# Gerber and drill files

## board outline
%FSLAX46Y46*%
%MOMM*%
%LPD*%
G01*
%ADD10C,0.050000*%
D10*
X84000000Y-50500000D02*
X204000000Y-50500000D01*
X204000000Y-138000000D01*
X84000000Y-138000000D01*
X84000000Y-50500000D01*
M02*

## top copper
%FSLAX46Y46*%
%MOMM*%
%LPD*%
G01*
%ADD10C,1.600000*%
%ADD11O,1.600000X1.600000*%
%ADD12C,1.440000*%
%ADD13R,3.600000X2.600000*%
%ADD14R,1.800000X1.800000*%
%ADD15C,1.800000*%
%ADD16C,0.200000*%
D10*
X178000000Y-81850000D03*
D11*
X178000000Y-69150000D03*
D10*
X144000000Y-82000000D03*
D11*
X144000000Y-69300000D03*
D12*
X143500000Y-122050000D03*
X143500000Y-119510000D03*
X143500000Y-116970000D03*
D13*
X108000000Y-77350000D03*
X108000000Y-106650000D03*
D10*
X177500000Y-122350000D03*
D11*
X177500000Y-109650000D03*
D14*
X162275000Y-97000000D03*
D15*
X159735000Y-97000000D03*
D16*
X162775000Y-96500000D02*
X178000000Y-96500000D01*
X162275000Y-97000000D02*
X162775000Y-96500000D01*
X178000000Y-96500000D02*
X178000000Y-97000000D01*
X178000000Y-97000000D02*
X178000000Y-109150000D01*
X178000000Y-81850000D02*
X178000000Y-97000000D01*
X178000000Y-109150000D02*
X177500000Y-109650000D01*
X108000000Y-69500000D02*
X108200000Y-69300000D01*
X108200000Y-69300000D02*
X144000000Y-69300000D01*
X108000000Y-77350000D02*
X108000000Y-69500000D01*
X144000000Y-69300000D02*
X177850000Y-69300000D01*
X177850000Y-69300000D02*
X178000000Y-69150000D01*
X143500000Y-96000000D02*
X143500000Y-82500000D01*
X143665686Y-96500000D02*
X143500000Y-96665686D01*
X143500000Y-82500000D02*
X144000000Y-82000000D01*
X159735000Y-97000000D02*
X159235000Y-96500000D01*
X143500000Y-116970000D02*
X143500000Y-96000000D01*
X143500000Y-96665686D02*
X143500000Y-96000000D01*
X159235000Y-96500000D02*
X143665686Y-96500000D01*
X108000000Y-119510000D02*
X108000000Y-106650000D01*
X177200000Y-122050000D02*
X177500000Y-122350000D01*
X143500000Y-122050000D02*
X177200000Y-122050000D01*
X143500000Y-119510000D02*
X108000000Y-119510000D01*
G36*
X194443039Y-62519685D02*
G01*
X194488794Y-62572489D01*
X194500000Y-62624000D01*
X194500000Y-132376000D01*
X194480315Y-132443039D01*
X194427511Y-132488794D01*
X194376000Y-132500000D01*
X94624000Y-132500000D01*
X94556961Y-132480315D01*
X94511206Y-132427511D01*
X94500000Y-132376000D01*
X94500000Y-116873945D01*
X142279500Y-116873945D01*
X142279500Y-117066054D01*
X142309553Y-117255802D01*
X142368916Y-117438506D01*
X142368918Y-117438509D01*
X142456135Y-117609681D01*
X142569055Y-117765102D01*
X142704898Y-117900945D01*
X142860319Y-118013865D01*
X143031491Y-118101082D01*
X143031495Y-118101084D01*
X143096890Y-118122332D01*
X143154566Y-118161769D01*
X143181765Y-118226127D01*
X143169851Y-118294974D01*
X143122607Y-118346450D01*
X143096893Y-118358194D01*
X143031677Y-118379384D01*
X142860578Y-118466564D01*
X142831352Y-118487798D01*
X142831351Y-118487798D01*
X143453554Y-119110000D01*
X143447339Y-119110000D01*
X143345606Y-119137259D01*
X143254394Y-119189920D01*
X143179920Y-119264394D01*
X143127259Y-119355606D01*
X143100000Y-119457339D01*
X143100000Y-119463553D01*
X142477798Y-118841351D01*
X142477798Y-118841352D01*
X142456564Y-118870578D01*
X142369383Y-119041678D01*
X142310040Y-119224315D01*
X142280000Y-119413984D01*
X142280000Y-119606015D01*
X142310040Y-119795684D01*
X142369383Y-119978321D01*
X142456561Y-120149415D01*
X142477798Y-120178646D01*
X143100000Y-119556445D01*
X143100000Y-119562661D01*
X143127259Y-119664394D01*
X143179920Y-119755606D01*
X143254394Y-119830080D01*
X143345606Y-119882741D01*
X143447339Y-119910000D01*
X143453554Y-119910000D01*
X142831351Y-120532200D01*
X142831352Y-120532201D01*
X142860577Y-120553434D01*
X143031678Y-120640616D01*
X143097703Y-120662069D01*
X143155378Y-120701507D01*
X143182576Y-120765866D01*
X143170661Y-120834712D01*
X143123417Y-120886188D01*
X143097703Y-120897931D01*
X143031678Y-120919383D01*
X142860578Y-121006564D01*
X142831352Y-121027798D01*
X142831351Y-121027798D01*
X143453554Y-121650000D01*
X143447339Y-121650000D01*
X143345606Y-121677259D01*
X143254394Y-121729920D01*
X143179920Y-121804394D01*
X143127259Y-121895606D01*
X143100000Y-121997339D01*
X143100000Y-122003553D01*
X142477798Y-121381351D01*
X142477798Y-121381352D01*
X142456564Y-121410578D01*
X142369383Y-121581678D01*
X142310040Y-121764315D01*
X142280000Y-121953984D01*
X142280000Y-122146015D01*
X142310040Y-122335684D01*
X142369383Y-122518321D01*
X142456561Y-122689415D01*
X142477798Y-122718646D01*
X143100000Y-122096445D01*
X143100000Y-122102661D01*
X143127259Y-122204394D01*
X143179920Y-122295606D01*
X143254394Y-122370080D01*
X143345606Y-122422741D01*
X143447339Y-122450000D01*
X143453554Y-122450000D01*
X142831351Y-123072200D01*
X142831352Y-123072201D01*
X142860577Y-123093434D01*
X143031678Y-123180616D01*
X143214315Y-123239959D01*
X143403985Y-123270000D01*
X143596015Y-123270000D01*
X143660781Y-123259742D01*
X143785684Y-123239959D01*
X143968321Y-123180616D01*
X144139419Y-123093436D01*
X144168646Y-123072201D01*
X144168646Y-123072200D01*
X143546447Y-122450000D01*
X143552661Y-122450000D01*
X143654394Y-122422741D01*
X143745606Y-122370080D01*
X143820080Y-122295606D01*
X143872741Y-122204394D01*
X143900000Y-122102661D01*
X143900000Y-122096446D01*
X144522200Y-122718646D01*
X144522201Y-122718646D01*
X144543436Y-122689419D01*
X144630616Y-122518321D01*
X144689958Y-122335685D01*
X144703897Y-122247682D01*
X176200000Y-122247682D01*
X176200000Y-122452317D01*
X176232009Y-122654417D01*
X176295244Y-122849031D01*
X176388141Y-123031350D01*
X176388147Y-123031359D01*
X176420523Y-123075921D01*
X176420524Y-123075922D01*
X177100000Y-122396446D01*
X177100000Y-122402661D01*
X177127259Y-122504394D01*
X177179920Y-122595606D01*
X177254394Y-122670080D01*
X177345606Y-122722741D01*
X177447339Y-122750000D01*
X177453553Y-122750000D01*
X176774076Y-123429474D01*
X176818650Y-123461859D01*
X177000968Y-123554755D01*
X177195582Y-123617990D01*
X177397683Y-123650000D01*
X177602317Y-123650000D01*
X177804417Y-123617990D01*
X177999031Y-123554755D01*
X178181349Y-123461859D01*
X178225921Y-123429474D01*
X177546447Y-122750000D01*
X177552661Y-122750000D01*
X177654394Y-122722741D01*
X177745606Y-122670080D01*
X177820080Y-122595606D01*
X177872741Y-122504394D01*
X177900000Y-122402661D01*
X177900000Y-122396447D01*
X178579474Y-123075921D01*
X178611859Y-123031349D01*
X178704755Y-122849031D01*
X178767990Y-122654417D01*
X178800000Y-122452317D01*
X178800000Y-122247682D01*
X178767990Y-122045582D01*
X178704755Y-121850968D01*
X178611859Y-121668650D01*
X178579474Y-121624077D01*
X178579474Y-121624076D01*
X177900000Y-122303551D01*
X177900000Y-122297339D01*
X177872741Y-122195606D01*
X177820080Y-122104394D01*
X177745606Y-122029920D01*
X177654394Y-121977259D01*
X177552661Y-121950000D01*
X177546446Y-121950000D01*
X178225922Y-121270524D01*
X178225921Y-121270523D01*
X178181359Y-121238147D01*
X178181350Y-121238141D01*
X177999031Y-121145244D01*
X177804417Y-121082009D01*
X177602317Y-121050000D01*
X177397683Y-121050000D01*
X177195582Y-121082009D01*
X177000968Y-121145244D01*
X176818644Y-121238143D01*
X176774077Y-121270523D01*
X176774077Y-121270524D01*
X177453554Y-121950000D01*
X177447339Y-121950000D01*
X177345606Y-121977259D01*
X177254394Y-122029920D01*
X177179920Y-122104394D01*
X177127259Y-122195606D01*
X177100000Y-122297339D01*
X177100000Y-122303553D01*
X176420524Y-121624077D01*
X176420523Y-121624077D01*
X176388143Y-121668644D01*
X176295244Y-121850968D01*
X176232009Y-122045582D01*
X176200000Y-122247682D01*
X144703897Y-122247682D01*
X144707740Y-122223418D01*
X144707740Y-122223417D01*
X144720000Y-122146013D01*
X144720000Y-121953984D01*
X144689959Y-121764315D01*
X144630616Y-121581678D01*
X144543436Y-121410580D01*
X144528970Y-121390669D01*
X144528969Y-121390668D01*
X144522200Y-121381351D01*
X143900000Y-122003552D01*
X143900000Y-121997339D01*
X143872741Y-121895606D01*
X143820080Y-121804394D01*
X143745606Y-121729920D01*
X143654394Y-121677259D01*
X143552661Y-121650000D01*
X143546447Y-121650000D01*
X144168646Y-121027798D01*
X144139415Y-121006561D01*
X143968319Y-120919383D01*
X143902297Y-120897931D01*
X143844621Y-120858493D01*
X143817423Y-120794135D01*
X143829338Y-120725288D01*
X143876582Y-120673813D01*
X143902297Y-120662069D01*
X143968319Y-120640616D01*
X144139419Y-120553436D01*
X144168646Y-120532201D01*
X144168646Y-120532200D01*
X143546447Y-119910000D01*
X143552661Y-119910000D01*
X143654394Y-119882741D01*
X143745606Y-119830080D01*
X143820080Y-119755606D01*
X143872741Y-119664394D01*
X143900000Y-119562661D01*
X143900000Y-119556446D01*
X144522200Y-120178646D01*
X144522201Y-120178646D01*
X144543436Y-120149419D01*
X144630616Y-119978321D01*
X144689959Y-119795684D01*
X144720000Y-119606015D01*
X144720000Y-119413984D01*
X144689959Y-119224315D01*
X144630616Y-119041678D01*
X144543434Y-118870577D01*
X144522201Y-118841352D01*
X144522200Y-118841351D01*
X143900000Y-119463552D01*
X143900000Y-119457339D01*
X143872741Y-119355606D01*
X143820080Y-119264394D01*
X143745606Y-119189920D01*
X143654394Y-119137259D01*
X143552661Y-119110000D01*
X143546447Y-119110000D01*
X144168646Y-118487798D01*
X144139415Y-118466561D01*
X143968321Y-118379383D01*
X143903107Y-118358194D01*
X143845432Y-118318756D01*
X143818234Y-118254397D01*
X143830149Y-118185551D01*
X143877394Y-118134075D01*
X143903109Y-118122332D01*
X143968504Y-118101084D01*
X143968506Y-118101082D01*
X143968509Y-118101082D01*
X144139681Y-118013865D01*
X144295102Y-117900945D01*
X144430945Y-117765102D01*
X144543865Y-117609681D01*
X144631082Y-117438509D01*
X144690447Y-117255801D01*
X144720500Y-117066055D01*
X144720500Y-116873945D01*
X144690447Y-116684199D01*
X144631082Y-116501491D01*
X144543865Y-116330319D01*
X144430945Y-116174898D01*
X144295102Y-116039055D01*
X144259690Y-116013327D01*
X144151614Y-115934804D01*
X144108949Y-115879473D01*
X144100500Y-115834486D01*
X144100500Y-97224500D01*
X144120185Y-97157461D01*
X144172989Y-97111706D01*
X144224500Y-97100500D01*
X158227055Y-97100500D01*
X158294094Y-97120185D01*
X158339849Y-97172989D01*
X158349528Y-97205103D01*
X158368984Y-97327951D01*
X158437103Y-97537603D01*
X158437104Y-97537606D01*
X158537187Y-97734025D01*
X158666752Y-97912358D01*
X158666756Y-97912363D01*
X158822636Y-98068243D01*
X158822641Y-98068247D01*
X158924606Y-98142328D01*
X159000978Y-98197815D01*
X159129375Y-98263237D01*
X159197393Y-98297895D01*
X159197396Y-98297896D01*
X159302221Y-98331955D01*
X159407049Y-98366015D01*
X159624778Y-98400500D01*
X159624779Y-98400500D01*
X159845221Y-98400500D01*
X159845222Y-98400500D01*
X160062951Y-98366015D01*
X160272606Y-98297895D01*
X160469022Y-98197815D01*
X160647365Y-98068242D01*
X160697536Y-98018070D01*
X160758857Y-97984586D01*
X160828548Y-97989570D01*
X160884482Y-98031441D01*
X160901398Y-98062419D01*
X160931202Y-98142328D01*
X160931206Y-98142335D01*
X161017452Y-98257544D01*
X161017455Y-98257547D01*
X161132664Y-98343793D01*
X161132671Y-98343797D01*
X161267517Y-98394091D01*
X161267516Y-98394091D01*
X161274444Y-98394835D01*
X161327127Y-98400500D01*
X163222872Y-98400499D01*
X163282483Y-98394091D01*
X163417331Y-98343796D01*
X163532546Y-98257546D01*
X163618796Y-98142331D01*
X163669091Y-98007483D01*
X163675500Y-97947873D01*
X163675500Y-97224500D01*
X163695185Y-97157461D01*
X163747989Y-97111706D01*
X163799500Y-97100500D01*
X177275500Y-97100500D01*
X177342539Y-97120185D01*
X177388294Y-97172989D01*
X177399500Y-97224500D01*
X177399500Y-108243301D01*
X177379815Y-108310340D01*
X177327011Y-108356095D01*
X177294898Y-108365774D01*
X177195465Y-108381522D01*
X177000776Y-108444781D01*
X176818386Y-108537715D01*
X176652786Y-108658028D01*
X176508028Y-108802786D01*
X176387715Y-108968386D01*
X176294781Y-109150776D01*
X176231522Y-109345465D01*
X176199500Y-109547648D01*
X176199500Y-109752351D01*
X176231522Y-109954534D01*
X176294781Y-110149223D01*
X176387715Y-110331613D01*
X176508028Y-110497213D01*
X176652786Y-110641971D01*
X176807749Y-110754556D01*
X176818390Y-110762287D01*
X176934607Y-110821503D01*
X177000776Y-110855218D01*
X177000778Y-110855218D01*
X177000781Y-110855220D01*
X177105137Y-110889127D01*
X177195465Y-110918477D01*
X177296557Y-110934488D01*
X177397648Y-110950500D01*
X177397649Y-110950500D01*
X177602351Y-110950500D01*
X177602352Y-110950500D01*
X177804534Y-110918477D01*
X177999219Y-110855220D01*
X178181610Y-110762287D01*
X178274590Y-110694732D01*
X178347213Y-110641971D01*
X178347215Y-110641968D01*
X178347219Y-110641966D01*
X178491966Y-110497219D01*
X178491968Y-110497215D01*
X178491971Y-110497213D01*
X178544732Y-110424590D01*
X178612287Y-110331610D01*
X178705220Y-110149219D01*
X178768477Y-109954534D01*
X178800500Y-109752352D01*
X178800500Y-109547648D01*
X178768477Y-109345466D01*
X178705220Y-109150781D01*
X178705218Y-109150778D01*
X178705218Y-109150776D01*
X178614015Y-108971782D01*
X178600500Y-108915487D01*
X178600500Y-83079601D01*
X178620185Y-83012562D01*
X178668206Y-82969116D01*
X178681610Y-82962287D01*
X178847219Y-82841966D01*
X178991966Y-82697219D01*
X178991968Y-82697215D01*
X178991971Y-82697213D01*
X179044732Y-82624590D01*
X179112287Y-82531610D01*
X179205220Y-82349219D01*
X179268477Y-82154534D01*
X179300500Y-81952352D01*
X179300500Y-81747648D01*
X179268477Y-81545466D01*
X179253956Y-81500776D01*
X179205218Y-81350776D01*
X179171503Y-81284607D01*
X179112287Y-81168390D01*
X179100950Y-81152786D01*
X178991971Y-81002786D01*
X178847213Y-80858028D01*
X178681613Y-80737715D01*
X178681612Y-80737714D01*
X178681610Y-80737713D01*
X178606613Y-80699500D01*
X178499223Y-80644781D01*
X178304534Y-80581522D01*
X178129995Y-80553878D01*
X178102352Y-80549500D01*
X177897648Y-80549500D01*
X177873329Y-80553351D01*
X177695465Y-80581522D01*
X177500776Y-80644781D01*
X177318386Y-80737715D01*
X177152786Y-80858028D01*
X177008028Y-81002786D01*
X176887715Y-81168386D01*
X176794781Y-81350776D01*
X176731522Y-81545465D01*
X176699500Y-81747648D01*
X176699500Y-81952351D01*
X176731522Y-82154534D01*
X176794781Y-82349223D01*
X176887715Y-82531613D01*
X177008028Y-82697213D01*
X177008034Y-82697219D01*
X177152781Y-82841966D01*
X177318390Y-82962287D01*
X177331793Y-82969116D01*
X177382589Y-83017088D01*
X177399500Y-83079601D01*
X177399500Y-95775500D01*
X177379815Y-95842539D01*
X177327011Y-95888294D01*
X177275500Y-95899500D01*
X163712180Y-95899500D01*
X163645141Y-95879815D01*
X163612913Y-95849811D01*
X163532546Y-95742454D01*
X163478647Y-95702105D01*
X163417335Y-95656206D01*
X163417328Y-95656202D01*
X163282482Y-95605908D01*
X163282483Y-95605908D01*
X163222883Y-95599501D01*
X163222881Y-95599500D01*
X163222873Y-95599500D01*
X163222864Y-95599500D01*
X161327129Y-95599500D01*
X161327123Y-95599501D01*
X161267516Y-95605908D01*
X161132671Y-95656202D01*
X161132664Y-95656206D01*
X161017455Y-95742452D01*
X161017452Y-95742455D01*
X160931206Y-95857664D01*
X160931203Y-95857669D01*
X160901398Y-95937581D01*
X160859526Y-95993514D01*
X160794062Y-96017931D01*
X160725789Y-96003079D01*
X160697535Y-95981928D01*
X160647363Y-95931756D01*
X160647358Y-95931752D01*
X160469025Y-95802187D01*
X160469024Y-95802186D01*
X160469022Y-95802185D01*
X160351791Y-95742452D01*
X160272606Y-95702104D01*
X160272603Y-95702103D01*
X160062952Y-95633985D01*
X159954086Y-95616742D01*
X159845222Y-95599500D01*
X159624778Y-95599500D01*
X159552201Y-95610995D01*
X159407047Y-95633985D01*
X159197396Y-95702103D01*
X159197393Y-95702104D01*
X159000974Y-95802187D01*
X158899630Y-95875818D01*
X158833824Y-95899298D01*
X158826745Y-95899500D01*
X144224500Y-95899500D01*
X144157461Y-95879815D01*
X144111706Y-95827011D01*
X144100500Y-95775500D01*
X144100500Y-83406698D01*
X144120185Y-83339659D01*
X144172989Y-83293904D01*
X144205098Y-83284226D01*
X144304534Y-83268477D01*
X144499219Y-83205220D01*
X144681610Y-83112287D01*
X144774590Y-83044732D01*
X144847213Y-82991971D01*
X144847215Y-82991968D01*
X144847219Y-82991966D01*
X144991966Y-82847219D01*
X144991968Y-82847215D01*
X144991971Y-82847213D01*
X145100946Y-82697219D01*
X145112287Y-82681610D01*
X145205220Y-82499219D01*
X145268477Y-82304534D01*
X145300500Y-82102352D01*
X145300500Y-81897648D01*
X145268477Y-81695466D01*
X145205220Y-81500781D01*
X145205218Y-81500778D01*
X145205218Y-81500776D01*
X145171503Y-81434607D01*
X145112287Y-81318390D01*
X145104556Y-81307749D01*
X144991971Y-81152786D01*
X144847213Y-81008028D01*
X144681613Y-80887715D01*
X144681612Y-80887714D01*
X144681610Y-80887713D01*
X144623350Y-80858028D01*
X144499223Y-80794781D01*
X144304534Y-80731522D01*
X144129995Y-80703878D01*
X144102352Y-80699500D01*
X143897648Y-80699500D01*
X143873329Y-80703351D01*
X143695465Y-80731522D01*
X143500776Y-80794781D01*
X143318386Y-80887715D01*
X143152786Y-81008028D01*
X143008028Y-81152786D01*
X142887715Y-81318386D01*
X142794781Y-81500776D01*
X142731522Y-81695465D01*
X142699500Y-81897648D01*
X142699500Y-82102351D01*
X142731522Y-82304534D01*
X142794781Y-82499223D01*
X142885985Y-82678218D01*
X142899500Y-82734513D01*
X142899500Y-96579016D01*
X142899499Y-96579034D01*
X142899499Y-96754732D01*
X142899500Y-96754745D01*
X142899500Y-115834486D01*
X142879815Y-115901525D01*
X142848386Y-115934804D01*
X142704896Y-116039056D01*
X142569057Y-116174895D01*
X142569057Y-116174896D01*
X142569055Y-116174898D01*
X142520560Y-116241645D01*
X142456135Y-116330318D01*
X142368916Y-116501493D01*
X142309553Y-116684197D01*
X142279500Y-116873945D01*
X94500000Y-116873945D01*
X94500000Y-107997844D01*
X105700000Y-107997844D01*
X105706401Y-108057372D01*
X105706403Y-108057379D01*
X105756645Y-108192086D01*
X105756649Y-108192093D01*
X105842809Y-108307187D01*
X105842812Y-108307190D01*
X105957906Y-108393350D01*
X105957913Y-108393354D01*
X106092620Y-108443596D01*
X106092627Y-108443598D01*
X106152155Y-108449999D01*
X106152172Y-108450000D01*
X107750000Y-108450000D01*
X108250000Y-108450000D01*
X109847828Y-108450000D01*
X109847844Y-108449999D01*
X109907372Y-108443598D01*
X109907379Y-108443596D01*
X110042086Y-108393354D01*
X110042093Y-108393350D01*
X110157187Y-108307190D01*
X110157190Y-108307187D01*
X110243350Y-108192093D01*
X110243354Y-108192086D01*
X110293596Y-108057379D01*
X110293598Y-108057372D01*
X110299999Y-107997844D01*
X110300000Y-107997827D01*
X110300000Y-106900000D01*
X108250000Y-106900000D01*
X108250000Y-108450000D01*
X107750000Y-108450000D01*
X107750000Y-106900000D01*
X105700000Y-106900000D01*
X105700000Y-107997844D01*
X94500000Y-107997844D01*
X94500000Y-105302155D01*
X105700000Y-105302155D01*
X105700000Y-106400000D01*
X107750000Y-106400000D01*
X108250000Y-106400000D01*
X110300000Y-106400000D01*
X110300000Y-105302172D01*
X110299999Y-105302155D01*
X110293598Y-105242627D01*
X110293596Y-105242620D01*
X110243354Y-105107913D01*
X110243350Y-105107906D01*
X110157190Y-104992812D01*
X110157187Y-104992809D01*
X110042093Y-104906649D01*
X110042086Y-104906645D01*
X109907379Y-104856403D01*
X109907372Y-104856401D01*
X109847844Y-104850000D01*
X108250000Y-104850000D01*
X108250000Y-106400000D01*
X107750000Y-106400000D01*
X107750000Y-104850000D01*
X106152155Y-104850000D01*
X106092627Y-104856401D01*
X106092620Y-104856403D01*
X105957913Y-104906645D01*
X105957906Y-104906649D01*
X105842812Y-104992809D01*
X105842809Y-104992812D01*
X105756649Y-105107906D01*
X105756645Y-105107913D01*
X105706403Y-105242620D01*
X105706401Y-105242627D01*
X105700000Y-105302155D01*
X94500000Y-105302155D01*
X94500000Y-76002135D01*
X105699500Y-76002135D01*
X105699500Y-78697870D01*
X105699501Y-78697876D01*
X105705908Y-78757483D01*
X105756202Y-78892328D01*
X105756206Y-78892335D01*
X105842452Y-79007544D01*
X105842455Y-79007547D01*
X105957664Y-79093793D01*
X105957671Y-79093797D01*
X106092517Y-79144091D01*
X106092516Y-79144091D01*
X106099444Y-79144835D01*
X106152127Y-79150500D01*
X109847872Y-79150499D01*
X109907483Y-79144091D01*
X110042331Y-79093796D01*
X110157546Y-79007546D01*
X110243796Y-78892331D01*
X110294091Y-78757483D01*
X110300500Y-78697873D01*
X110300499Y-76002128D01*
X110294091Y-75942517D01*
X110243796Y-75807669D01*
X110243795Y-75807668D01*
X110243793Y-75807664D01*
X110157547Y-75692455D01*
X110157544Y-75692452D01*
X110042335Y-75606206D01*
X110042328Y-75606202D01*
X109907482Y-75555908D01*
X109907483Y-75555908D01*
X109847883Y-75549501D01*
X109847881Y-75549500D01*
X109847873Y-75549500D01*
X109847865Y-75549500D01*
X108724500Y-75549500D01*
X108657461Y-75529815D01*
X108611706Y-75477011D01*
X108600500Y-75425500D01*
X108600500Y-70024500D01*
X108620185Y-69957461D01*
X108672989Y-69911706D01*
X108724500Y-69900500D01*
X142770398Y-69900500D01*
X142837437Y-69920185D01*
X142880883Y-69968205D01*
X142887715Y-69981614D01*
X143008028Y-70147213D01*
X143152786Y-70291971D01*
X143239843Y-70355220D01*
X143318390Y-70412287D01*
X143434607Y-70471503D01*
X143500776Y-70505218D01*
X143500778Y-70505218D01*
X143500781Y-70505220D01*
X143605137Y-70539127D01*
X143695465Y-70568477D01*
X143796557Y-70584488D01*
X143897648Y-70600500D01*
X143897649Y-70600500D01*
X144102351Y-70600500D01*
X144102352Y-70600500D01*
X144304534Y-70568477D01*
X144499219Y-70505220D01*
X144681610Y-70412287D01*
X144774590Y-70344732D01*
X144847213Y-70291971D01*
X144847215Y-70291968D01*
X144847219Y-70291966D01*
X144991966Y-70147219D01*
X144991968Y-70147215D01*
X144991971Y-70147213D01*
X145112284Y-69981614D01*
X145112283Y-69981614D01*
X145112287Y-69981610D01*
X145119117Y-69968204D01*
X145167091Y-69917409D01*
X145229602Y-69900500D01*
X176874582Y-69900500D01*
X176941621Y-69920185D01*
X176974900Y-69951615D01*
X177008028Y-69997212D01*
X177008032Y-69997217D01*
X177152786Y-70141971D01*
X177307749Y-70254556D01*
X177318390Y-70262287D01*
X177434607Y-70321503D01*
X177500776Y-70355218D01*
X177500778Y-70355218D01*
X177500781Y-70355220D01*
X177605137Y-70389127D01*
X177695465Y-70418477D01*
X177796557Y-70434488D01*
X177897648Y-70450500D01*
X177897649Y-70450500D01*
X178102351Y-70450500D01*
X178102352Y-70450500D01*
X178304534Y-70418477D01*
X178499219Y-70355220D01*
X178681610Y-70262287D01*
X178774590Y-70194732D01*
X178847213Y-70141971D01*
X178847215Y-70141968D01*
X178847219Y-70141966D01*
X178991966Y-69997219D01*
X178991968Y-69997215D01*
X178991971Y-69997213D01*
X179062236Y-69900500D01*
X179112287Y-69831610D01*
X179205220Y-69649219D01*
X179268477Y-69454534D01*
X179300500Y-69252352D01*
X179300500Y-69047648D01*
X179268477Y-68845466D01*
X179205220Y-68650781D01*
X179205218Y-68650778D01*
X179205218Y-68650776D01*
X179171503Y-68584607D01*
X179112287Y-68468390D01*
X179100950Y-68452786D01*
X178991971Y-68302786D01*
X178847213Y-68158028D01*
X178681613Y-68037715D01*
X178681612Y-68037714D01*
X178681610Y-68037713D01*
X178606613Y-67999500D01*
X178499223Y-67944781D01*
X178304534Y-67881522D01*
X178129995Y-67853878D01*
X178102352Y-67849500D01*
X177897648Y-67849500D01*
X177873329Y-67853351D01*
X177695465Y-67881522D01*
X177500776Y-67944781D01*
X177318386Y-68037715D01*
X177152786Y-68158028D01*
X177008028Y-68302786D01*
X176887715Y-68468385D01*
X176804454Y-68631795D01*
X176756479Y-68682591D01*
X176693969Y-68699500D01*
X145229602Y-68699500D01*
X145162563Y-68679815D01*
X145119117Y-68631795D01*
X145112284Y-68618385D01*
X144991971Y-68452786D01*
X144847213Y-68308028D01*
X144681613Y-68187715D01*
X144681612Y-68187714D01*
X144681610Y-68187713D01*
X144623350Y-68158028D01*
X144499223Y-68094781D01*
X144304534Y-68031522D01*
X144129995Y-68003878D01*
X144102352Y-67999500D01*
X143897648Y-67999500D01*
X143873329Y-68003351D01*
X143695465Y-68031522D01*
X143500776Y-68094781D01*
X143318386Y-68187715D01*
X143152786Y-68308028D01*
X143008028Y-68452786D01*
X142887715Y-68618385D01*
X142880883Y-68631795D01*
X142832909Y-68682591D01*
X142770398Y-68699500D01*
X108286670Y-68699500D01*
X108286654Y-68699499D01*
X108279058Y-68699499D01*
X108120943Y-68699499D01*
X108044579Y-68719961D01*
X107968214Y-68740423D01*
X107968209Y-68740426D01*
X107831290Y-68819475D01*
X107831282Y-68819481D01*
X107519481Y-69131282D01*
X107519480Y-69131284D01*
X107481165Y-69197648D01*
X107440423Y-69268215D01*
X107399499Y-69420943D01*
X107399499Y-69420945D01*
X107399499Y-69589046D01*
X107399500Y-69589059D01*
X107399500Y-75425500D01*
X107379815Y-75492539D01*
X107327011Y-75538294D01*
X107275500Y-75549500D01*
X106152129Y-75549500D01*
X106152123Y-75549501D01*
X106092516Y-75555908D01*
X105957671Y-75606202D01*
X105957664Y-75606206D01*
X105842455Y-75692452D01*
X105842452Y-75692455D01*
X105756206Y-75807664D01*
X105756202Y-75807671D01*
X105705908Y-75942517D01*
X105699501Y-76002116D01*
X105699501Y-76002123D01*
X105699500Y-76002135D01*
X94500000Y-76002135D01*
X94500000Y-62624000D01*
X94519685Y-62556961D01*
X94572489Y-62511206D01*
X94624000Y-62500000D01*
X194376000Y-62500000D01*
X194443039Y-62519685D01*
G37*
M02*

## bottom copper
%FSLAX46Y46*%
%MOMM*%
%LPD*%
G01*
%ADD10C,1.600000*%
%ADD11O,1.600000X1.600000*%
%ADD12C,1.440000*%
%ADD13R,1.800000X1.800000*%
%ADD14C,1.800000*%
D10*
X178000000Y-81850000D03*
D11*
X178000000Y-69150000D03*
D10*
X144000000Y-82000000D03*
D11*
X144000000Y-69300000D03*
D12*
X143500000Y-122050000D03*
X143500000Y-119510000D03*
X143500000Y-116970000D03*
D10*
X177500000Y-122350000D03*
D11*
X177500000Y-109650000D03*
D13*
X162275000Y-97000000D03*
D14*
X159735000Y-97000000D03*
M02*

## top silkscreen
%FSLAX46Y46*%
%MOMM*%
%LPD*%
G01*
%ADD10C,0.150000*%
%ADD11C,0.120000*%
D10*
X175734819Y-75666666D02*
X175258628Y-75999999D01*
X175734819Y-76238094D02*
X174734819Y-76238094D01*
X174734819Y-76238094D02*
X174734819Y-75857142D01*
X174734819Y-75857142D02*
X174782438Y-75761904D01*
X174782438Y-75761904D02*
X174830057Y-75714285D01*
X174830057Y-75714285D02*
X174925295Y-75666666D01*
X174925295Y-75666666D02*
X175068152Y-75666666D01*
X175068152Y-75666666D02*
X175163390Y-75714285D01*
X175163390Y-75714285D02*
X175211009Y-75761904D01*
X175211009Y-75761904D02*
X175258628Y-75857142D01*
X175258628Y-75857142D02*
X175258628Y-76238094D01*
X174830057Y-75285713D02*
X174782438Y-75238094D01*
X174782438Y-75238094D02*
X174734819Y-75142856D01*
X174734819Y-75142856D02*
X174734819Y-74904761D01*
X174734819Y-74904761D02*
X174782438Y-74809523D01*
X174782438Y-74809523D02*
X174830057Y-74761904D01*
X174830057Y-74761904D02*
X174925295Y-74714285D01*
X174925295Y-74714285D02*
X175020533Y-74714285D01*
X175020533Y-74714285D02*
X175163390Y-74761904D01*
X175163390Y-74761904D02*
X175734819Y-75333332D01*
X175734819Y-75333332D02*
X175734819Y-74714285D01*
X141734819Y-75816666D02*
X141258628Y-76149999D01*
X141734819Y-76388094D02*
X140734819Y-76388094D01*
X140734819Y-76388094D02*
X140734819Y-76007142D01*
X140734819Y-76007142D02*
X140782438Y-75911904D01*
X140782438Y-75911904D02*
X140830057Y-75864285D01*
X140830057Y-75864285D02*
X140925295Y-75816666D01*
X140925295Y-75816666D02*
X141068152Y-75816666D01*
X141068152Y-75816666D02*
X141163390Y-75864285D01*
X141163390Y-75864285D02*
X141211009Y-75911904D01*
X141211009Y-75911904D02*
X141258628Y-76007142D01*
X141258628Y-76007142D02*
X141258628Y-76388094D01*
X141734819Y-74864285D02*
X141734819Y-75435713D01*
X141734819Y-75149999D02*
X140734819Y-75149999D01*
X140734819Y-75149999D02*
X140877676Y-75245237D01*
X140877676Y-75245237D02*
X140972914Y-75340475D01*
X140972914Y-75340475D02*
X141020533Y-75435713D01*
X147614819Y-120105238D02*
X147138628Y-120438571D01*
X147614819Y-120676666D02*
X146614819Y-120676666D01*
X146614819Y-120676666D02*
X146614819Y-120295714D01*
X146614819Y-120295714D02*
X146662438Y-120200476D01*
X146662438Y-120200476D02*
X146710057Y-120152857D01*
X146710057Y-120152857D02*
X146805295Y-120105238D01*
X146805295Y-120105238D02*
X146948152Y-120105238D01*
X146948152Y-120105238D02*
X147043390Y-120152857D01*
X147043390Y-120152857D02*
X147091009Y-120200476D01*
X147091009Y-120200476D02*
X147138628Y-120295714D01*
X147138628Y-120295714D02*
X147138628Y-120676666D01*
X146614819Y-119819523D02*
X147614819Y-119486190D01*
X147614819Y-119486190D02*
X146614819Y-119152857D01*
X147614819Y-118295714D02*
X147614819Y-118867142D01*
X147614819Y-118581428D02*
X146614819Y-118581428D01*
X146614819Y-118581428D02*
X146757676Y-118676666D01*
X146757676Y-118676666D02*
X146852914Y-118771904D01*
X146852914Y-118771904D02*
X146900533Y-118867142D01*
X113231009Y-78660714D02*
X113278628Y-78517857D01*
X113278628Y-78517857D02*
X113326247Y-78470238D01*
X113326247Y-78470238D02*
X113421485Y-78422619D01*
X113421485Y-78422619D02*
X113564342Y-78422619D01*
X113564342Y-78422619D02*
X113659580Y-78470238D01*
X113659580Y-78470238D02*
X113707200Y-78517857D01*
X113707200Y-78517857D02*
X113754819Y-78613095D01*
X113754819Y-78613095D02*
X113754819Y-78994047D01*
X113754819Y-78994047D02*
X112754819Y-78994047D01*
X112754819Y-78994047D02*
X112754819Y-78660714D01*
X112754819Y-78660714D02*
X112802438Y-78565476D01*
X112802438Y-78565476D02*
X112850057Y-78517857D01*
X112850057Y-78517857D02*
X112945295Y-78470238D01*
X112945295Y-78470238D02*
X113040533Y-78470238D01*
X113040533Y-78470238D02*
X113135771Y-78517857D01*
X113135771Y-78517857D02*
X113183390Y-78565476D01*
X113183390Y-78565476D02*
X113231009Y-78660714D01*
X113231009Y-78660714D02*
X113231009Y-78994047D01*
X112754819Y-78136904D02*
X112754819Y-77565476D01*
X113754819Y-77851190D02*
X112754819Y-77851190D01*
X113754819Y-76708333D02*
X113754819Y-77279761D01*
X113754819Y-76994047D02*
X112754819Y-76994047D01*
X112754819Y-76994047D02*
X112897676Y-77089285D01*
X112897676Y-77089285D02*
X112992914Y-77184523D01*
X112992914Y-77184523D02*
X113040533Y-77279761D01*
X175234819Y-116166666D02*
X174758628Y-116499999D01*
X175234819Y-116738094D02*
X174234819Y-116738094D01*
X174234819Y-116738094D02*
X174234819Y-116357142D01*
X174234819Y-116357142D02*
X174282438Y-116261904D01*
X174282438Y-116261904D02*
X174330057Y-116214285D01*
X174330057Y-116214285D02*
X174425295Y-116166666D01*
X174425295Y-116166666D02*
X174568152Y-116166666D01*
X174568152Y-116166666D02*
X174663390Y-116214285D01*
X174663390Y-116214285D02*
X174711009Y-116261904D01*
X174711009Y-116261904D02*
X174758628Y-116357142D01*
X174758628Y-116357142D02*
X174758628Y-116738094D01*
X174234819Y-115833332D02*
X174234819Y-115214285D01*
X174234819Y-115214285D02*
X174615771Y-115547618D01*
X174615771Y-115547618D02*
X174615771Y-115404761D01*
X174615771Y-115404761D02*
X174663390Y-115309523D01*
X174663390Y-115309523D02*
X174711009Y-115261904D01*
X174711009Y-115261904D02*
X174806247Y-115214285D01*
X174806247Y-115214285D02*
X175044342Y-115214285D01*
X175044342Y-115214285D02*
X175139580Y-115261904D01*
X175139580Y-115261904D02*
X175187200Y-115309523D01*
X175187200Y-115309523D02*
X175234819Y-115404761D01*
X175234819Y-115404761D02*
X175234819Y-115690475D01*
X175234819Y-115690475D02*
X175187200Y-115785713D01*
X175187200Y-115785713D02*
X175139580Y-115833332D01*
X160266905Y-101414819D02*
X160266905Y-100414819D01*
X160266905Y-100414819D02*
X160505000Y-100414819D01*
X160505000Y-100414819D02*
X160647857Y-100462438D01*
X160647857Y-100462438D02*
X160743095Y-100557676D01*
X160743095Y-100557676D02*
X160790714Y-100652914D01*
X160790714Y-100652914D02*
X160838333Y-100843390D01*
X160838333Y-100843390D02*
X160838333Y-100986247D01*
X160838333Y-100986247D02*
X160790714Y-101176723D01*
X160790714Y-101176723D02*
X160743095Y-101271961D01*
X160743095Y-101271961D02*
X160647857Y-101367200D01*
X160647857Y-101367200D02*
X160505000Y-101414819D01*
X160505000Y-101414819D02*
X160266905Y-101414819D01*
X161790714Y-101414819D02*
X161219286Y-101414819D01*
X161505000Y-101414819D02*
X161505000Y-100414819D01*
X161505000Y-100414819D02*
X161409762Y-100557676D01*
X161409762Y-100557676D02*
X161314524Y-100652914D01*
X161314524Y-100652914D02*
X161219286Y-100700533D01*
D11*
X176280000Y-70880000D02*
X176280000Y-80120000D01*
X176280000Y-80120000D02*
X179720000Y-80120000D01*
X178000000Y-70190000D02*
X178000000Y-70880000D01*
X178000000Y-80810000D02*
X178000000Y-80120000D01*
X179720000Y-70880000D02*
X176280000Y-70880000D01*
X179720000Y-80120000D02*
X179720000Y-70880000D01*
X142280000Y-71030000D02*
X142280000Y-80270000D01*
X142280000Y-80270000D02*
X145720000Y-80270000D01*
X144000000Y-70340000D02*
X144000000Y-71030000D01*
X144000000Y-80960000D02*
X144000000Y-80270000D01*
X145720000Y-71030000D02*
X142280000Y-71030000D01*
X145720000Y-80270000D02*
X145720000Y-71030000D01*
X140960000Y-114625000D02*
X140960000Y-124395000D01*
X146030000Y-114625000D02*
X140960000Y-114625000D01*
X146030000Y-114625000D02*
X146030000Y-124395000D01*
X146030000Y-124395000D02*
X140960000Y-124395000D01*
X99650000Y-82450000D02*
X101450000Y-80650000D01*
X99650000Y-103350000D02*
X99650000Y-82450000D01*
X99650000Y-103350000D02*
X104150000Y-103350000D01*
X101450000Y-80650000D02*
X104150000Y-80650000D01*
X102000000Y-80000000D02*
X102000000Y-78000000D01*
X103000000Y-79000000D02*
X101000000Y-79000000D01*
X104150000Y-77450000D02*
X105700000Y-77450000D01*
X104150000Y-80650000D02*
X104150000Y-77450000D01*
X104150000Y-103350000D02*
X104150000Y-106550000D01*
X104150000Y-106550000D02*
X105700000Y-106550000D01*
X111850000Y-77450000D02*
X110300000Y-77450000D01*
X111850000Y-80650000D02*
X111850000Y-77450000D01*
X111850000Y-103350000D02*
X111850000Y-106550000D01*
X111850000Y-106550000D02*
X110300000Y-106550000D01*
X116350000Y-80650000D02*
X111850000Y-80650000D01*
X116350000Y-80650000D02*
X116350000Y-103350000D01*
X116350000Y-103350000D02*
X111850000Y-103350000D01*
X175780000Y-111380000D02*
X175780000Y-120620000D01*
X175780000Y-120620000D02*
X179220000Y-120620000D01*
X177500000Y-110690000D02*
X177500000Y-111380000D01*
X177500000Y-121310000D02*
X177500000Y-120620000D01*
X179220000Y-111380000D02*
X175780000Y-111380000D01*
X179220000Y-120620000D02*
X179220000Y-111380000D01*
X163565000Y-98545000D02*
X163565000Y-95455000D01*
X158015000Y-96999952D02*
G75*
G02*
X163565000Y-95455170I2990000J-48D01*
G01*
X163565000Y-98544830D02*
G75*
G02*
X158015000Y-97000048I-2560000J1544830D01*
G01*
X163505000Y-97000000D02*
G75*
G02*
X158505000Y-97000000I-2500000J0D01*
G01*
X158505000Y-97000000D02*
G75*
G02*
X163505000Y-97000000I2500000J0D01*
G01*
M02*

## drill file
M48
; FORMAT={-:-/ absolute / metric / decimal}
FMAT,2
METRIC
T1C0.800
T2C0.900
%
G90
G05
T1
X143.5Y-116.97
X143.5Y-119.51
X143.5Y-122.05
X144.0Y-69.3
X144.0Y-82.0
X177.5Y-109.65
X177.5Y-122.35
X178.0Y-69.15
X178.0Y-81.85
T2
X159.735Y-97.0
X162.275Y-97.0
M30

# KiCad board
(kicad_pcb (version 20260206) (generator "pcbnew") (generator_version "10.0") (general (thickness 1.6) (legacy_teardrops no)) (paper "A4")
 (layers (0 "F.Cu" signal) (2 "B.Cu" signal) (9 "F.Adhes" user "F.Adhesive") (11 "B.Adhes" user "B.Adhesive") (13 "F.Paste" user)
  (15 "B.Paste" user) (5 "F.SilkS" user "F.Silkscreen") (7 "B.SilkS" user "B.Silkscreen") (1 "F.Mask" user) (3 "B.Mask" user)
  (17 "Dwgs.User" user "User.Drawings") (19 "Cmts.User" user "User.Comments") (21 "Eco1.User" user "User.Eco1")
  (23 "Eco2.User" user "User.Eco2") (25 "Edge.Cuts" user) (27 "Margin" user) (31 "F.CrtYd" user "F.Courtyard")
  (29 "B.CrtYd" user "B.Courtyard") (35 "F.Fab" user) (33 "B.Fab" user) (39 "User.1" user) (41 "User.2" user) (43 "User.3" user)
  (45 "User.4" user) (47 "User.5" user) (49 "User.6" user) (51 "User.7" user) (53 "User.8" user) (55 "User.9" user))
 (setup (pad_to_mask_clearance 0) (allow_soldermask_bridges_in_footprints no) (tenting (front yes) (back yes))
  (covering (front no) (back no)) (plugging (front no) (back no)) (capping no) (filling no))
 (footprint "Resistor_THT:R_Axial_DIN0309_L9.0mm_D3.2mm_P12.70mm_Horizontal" (layer "F.Cu") (at 178 81.85 90)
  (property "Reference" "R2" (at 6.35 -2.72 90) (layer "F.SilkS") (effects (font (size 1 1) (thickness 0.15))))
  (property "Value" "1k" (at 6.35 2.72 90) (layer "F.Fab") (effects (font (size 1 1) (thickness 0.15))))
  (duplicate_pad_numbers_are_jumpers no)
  (fp_line (start 10.97 -1.72) (end 1.73 -1.72) (stroke (width 0.12) (type solid)) (layer "F.SilkS"))
  (fp_line (start 1.73 -1.72) (end 1.73 1.72) (stroke (width 0.12) (type solid)) (layer "F.SilkS"))
  (fp_line (start 11.66 0) (end 10.97 0) (stroke (width 0.12) (type solid)) (layer "F.SilkS"))
  (fp_line (start 1.04 0) (end 1.73 0) (stroke (width 0.12) (type solid)) (layer "F.SilkS"))
  (fp_line (start 10.97 1.72) (end 10.97 -1.72) (stroke (width 0.12) (type solid)) (layer "F.SilkS"))
  (fp_line (start 1.73 1.72) (end 10.97 1.72) (stroke (width 0.12) (type solid)) (layer "F.SilkS"))
  (pad "1" thru_hole circle (at 0 0 90) (size 1.6 1.6) (drill 0.8) (layers "*.Cu" "*.Mask") (remove_unused_layers no) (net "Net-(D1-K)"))
  (pad "2" thru_hole oval (at 12.7 0 90) (size 1.6 1.6) (drill 0.8) (layers "*.Cu" "*.Mask") (remove_unused_layers no) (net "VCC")))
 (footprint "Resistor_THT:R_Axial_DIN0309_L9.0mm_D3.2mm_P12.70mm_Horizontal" (layer "F.Cu") (at 144 82 90)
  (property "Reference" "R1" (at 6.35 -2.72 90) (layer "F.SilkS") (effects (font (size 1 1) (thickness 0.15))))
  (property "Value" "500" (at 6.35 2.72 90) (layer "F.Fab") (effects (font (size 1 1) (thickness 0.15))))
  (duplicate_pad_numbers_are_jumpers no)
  (fp_line (start 10.97 -1.72) (end 1.73 -1.72) (stroke (width 0.12) (type solid)) (layer "F.SilkS"))
  (fp_line (start 1.73 -1.72) (end 1.73 1.72) (stroke (width 0.12) (type solid)) (layer "F.SilkS"))
  (fp_line (start 11.66 0) (end 10.97 0) (stroke (width 0.12) (type solid)) (layer "F.SilkS"))
  (fp_line (start 1.04 0) (end 1.73 0) (stroke (width 0.12) (type solid)) (layer "F.SilkS"))
  (fp_line (start 10.97 1.72) (end 10.97 -1.72) (stroke (width 0.12) (type solid)) (layer "F.SilkS"))
  (fp_line (start 1.73 1.72) (end 10.97 1.72) (stroke (width 0.12) (type solid)) (layer "F.SilkS"))
  (pad "1" thru_hole circle (at 0 0 90) (size 1.6 1.6) (drill 0.8) (layers "*.Cu" "*.Mask") (remove_unused_layers no) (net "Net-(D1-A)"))
  (pad "2" thru_hole oval (at 12.7 0 90) (size 1.6 1.6) (drill 0.8) (layers "*.Cu" "*.Mask") (remove_unused_layers no) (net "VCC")))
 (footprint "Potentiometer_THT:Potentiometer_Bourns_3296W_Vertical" (layer "F.Cu") (at 143.5 122.05 -90)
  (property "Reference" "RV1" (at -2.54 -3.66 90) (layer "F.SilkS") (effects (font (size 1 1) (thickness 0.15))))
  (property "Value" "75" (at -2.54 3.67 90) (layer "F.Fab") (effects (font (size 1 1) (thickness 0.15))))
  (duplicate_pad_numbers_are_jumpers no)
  (fp_line (start -7.425 2.54) (end 2.345 2.54) (stroke (width 0.12) (type solid)) (layer "F.SilkS"))
  (fp_line (start -7.425 -2.53) (end -7.425 2.54) (stroke (width 0.12) (type solid)) (layer "F.SilkS"))
  (fp_line (start -7.425 -2.53) (end 2.345 -2.53) (stroke (width 0.12) (type solid)) (layer "F.SilkS"))
  (fp_line (start 2.345 -2.53) (end 2.345 2.54) (stroke (width 0.12) (type solid)) (layer "F.SilkS"))
  (pad "1" thru_hole circle (at 0 0 270) (size 1.44 1.44) (drill 0.8) (layers "*.Cu" "*.Mask") (remove_unused_layers no) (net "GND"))
  (pad "2" thru_hole circle (at -2.54 0 270) (size 1.44 1.44) (drill 0.8) (layers "*.Cu" "*.Mask") (remove_unused_layers no) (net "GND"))
  (pad "3" thru_hole circle (at -5.08 0 270) (size 1.44 1.44) (drill 0.8) (layers "*.Cu" "*.Mask") (remove_unused_layers no)
   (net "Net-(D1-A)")))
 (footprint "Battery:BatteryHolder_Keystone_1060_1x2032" (layer "F.Cu") (at 108 92 -90)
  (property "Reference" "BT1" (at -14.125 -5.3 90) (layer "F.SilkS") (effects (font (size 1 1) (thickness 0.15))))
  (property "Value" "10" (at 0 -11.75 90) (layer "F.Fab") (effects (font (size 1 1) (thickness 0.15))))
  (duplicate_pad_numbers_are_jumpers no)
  (fp_line (start -9.55 8.35) (end -11.35 6.55) (stroke (width 0.12) (type solid)) (layer "F.SilkS"))
  (fp_line (start 11.35 8.35) (end -9.55 8.35) (stroke (width 0.12) (type solid)) (layer "F.SilkS"))
  (fp_line (start 11.35 8.35) (end 11.35 3.85) (stroke (width 0.12) (type solid)) (layer "F.SilkS"))
  (fp_line (start -11.35 6.55) (end -11.35 3.85) (stroke (width 0.12) (type solid)) (layer "F.SilkS"))
  (fp_line (start -12 6) (end -14 6) (stroke (width 0.12) (type solid)) (layer "F.SilkS"))
  (fp_line (start -13 5) (end -13 7) (stroke (width 0.12) (type solid)) (layer "F.SilkS"))
  (fp_line (start -14.55 3.85) (end -14.55 2.3) (stroke (width 0.12) (type solid)) (layer "F.SilkS"))
  (fp_line (start -11.35 3.85) (end -14.55 3.85) (stroke (width 0.12) (type solid)) (layer "F.SilkS"))
  (fp_line (start 11.35 3.85) (end 14.55 3.85) (stroke (width 0.12) (type solid)) (layer "F.SilkS"))
  (fp_line (start 14.55 3.85) (end 14.55 2.3) (stroke (width 0.12) (type solid)) (layer "F.SilkS"))
  (fp_line (start -14.55 -3.85) (end -14.55 -2.3) (stroke (width 0.12) (type solid)) (layer "F.SilkS"))
  (fp_line (start -11.35 -3.85) (end -14.55 -3.85) (stroke (width 0.12) (type solid)) (layer "F.SilkS"))
  (fp_line (start 11.35 -3.85) (end 14.55 -3.85) (stroke (width 0.12) (type solid)) (layer "F.SilkS"))
  (fp_line (start 14.55 -3.85) (end 14.55 -2.3) (stroke (width 0.12) (type solid)) (layer "F.SilkS"))
  (fp_line (start -11.35 -8.35) (end -11.35 -3.85) (stroke (width 0.12) (type solid)) (layer "F.SilkS"))
  (fp_line (start -11.35 -8.35) (end 11.35 -8.35) (stroke (width 0.12) (type solid)) (layer "F.SilkS"))
  (fp_line (start 11.35 -8.35) (end 11.35 -3.85) (stroke (width 0.12) (type solid)) (layer "F.SilkS"))
  (pad "1" smd rect (at -14.65 0 90) (size 2.6 3.6) (layers "F.Cu" "F.Mask" "F.Paste") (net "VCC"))
  (pad "2" smd rect (at 14.65 0 90) (size 2.6 3.6) (layers "F.Cu" "F.Mask" "F.Paste") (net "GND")))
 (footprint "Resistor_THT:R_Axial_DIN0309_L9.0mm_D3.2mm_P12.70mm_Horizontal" (layer "F.Cu") (at 177.5 122.35 90)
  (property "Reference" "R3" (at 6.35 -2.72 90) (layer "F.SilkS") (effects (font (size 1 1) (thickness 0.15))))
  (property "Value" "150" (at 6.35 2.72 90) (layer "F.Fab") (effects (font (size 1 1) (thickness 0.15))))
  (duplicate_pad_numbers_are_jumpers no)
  (fp_line (start 10.97 -1.72) (end 1.73 -1.72) (stroke (width 0.12) (type solid)) (layer "F.SilkS"))
  (fp_line (start 1.73 -1.72) (end 1.73 1.72) (stroke (width 0.12) (type solid)) (layer "F.SilkS"))
  (fp_line (start 11.66 0) (end 10.97 0) (stroke (width 0.12) (type solid)) (layer "F.SilkS"))
  (fp_line (start 1.04 0) (end 1.73 0) (stroke (width 0.12) (type solid)) (layer "F.SilkS"))
  (fp_line (start 10.97 1.72) (end 10.97 -1.72) (stroke (width 0.12) (type solid)) (layer "F.SilkS"))
  (fp_line (start 1.73 1.72) (end 10.97 1.72) (stroke (width 0.12) (type solid)) (layer "F.SilkS"))
  (pad "1" thru_hole circle (at 0 0 90) (size 1.6 1.6) (drill 0.8) (layers "*.Cu" "*.Mask") (remove_unused_layers no) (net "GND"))
  (pad "2" thru_hole oval (at 12.7 0 90) (size 1.6 1.6) (drill 0.8) (layers "*.Cu" "*.Mask") (remove_unused_layers no) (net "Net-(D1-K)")))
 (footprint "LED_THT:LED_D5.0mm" (layer "F.Cu") (at 162.275 97 180)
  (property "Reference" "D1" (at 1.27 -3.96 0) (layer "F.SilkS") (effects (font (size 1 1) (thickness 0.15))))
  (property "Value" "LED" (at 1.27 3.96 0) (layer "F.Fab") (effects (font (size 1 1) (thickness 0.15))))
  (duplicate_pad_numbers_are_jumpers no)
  (fp_line (start -1.29 -1.545) (end -1.29 1.545) (stroke (width 0.12) (type solid)) (layer "F.SilkS"))
  (fp_arc (start 4.26 0.000048) (mid 2.071756 2.880501) (end -1.29 1.54483) (stroke (width 0.12) (type solid)) (layer "F.SilkS"))
  (fp_arc (start -1.29 -1.54483) (mid 2.071756 -2.880501) (end 4.26 -0.000048) (stroke (width 0.12) (type solid)) (layer "F.SilkS"))
  (fp_circle (center 1.27 0) (end 3.77 0) (stroke (width 0.12) (type solid)) (fill no) (layer "F.SilkS"))
  (pad "1" thru_hole rect (at 0 0 180) (size 1.8 1.8) (drill 0.9) (layers "*.Cu" "*.Mask") (remove_unused_layers no) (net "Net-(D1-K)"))
  (pad "2" thru_hole circle (at 2.54 0 180) (size 1.8 1.8) (drill 0.9) (layers "*.Cu" "*.Mask") (remove_unused_layers no) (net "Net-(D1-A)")))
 (gr_rect (start 84 50.5) (end 204 138) (stroke (width 0.05) (type default)) (fill no) (layer "Edge.Cuts"))
 (segment (start 162.775 96.5) (end 178 96.5) (width 0.2) (layer "F.Cu") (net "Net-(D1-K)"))
 (segment (start 162.275 97) (end 162.775 96.5) (width 0.2) (layer "F.Cu") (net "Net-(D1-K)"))
 (segment (start 178 96.5) (end 178 97) (width 0.2) (layer "F.Cu") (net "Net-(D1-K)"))
 (segment (start 178 97) (end 178 109.15) (width 0.2) (layer "F.Cu") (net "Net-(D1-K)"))
 (segment (start 178 81.85) (end 178 97) (width 0.2) (layer "F.Cu") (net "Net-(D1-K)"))
 (segment (start 178 109.15) (end 177.5 109.65) (width 0.2) (layer "F.Cu") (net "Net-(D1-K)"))
 (segment (start 108 69.5) (end 108.2 69.3) (width 0.2) (layer "F.Cu") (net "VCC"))
 (segment (start 108.2 69.3) (end 144 69.3) (width 0.2) (layer "F.Cu") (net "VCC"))
 (segment (start 108 77.35) (end 108 69.5) (width 0.2) (layer "F.Cu") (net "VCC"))
 (segment (start 144 69.3) (end 177.85 69.3) (width 0.2) (layer "F.Cu") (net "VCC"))
 (segment (start 177.85 69.3) (end 178 69.15) (width 0.2) (layer "F.Cu") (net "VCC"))
 (segment (start 143.5 96) (end 143.5 82.5) (width 0.2) (layer "F.Cu") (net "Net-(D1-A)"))
 (segment (start 143.665686 96.5) (end 143.5 96.665686) (width 0.2) (layer "F.Cu") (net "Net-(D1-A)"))
 (segment (start 143.5 82.5) (end 144 82) (width 0.2) (layer "F.Cu") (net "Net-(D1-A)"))
 (segment (start 159.735 97) (end 159.235 96.5) (width 0.2) (layer "F.Cu") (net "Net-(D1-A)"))
 (segment (start 143.5 116.97) (end 143.5 96) (width 0.2) (layer "F.Cu") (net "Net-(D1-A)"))
 (segment (start 143.5 96.665686) (end 143.5 96) (width 0.2) (layer "F.Cu") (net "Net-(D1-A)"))
 (segment (start 159.235 96.5) (end 143.665686 96.5) (width 0.2) (layer "F.Cu") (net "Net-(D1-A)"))
 (segment (start 108 119.51) (end 108 106.65) (width 0.2) (layer "F.Cu") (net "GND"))
 (segment (start 177.2 122.05) (end 177.5 122.35) (width 0.2) (layer "F.Cu") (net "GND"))
 (segment (start 143.5 122.05) (end 177.2 122.05) (width 0.2) (layer "F.Cu") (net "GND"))
 (segment (start 143.5 119.51) (end 108 119.51) (width 0.2) (layer "F.Cu") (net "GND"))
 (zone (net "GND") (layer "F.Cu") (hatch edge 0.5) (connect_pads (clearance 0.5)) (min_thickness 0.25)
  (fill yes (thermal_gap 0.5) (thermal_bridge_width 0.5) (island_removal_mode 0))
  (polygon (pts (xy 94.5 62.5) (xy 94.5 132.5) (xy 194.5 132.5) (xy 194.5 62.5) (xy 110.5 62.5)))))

